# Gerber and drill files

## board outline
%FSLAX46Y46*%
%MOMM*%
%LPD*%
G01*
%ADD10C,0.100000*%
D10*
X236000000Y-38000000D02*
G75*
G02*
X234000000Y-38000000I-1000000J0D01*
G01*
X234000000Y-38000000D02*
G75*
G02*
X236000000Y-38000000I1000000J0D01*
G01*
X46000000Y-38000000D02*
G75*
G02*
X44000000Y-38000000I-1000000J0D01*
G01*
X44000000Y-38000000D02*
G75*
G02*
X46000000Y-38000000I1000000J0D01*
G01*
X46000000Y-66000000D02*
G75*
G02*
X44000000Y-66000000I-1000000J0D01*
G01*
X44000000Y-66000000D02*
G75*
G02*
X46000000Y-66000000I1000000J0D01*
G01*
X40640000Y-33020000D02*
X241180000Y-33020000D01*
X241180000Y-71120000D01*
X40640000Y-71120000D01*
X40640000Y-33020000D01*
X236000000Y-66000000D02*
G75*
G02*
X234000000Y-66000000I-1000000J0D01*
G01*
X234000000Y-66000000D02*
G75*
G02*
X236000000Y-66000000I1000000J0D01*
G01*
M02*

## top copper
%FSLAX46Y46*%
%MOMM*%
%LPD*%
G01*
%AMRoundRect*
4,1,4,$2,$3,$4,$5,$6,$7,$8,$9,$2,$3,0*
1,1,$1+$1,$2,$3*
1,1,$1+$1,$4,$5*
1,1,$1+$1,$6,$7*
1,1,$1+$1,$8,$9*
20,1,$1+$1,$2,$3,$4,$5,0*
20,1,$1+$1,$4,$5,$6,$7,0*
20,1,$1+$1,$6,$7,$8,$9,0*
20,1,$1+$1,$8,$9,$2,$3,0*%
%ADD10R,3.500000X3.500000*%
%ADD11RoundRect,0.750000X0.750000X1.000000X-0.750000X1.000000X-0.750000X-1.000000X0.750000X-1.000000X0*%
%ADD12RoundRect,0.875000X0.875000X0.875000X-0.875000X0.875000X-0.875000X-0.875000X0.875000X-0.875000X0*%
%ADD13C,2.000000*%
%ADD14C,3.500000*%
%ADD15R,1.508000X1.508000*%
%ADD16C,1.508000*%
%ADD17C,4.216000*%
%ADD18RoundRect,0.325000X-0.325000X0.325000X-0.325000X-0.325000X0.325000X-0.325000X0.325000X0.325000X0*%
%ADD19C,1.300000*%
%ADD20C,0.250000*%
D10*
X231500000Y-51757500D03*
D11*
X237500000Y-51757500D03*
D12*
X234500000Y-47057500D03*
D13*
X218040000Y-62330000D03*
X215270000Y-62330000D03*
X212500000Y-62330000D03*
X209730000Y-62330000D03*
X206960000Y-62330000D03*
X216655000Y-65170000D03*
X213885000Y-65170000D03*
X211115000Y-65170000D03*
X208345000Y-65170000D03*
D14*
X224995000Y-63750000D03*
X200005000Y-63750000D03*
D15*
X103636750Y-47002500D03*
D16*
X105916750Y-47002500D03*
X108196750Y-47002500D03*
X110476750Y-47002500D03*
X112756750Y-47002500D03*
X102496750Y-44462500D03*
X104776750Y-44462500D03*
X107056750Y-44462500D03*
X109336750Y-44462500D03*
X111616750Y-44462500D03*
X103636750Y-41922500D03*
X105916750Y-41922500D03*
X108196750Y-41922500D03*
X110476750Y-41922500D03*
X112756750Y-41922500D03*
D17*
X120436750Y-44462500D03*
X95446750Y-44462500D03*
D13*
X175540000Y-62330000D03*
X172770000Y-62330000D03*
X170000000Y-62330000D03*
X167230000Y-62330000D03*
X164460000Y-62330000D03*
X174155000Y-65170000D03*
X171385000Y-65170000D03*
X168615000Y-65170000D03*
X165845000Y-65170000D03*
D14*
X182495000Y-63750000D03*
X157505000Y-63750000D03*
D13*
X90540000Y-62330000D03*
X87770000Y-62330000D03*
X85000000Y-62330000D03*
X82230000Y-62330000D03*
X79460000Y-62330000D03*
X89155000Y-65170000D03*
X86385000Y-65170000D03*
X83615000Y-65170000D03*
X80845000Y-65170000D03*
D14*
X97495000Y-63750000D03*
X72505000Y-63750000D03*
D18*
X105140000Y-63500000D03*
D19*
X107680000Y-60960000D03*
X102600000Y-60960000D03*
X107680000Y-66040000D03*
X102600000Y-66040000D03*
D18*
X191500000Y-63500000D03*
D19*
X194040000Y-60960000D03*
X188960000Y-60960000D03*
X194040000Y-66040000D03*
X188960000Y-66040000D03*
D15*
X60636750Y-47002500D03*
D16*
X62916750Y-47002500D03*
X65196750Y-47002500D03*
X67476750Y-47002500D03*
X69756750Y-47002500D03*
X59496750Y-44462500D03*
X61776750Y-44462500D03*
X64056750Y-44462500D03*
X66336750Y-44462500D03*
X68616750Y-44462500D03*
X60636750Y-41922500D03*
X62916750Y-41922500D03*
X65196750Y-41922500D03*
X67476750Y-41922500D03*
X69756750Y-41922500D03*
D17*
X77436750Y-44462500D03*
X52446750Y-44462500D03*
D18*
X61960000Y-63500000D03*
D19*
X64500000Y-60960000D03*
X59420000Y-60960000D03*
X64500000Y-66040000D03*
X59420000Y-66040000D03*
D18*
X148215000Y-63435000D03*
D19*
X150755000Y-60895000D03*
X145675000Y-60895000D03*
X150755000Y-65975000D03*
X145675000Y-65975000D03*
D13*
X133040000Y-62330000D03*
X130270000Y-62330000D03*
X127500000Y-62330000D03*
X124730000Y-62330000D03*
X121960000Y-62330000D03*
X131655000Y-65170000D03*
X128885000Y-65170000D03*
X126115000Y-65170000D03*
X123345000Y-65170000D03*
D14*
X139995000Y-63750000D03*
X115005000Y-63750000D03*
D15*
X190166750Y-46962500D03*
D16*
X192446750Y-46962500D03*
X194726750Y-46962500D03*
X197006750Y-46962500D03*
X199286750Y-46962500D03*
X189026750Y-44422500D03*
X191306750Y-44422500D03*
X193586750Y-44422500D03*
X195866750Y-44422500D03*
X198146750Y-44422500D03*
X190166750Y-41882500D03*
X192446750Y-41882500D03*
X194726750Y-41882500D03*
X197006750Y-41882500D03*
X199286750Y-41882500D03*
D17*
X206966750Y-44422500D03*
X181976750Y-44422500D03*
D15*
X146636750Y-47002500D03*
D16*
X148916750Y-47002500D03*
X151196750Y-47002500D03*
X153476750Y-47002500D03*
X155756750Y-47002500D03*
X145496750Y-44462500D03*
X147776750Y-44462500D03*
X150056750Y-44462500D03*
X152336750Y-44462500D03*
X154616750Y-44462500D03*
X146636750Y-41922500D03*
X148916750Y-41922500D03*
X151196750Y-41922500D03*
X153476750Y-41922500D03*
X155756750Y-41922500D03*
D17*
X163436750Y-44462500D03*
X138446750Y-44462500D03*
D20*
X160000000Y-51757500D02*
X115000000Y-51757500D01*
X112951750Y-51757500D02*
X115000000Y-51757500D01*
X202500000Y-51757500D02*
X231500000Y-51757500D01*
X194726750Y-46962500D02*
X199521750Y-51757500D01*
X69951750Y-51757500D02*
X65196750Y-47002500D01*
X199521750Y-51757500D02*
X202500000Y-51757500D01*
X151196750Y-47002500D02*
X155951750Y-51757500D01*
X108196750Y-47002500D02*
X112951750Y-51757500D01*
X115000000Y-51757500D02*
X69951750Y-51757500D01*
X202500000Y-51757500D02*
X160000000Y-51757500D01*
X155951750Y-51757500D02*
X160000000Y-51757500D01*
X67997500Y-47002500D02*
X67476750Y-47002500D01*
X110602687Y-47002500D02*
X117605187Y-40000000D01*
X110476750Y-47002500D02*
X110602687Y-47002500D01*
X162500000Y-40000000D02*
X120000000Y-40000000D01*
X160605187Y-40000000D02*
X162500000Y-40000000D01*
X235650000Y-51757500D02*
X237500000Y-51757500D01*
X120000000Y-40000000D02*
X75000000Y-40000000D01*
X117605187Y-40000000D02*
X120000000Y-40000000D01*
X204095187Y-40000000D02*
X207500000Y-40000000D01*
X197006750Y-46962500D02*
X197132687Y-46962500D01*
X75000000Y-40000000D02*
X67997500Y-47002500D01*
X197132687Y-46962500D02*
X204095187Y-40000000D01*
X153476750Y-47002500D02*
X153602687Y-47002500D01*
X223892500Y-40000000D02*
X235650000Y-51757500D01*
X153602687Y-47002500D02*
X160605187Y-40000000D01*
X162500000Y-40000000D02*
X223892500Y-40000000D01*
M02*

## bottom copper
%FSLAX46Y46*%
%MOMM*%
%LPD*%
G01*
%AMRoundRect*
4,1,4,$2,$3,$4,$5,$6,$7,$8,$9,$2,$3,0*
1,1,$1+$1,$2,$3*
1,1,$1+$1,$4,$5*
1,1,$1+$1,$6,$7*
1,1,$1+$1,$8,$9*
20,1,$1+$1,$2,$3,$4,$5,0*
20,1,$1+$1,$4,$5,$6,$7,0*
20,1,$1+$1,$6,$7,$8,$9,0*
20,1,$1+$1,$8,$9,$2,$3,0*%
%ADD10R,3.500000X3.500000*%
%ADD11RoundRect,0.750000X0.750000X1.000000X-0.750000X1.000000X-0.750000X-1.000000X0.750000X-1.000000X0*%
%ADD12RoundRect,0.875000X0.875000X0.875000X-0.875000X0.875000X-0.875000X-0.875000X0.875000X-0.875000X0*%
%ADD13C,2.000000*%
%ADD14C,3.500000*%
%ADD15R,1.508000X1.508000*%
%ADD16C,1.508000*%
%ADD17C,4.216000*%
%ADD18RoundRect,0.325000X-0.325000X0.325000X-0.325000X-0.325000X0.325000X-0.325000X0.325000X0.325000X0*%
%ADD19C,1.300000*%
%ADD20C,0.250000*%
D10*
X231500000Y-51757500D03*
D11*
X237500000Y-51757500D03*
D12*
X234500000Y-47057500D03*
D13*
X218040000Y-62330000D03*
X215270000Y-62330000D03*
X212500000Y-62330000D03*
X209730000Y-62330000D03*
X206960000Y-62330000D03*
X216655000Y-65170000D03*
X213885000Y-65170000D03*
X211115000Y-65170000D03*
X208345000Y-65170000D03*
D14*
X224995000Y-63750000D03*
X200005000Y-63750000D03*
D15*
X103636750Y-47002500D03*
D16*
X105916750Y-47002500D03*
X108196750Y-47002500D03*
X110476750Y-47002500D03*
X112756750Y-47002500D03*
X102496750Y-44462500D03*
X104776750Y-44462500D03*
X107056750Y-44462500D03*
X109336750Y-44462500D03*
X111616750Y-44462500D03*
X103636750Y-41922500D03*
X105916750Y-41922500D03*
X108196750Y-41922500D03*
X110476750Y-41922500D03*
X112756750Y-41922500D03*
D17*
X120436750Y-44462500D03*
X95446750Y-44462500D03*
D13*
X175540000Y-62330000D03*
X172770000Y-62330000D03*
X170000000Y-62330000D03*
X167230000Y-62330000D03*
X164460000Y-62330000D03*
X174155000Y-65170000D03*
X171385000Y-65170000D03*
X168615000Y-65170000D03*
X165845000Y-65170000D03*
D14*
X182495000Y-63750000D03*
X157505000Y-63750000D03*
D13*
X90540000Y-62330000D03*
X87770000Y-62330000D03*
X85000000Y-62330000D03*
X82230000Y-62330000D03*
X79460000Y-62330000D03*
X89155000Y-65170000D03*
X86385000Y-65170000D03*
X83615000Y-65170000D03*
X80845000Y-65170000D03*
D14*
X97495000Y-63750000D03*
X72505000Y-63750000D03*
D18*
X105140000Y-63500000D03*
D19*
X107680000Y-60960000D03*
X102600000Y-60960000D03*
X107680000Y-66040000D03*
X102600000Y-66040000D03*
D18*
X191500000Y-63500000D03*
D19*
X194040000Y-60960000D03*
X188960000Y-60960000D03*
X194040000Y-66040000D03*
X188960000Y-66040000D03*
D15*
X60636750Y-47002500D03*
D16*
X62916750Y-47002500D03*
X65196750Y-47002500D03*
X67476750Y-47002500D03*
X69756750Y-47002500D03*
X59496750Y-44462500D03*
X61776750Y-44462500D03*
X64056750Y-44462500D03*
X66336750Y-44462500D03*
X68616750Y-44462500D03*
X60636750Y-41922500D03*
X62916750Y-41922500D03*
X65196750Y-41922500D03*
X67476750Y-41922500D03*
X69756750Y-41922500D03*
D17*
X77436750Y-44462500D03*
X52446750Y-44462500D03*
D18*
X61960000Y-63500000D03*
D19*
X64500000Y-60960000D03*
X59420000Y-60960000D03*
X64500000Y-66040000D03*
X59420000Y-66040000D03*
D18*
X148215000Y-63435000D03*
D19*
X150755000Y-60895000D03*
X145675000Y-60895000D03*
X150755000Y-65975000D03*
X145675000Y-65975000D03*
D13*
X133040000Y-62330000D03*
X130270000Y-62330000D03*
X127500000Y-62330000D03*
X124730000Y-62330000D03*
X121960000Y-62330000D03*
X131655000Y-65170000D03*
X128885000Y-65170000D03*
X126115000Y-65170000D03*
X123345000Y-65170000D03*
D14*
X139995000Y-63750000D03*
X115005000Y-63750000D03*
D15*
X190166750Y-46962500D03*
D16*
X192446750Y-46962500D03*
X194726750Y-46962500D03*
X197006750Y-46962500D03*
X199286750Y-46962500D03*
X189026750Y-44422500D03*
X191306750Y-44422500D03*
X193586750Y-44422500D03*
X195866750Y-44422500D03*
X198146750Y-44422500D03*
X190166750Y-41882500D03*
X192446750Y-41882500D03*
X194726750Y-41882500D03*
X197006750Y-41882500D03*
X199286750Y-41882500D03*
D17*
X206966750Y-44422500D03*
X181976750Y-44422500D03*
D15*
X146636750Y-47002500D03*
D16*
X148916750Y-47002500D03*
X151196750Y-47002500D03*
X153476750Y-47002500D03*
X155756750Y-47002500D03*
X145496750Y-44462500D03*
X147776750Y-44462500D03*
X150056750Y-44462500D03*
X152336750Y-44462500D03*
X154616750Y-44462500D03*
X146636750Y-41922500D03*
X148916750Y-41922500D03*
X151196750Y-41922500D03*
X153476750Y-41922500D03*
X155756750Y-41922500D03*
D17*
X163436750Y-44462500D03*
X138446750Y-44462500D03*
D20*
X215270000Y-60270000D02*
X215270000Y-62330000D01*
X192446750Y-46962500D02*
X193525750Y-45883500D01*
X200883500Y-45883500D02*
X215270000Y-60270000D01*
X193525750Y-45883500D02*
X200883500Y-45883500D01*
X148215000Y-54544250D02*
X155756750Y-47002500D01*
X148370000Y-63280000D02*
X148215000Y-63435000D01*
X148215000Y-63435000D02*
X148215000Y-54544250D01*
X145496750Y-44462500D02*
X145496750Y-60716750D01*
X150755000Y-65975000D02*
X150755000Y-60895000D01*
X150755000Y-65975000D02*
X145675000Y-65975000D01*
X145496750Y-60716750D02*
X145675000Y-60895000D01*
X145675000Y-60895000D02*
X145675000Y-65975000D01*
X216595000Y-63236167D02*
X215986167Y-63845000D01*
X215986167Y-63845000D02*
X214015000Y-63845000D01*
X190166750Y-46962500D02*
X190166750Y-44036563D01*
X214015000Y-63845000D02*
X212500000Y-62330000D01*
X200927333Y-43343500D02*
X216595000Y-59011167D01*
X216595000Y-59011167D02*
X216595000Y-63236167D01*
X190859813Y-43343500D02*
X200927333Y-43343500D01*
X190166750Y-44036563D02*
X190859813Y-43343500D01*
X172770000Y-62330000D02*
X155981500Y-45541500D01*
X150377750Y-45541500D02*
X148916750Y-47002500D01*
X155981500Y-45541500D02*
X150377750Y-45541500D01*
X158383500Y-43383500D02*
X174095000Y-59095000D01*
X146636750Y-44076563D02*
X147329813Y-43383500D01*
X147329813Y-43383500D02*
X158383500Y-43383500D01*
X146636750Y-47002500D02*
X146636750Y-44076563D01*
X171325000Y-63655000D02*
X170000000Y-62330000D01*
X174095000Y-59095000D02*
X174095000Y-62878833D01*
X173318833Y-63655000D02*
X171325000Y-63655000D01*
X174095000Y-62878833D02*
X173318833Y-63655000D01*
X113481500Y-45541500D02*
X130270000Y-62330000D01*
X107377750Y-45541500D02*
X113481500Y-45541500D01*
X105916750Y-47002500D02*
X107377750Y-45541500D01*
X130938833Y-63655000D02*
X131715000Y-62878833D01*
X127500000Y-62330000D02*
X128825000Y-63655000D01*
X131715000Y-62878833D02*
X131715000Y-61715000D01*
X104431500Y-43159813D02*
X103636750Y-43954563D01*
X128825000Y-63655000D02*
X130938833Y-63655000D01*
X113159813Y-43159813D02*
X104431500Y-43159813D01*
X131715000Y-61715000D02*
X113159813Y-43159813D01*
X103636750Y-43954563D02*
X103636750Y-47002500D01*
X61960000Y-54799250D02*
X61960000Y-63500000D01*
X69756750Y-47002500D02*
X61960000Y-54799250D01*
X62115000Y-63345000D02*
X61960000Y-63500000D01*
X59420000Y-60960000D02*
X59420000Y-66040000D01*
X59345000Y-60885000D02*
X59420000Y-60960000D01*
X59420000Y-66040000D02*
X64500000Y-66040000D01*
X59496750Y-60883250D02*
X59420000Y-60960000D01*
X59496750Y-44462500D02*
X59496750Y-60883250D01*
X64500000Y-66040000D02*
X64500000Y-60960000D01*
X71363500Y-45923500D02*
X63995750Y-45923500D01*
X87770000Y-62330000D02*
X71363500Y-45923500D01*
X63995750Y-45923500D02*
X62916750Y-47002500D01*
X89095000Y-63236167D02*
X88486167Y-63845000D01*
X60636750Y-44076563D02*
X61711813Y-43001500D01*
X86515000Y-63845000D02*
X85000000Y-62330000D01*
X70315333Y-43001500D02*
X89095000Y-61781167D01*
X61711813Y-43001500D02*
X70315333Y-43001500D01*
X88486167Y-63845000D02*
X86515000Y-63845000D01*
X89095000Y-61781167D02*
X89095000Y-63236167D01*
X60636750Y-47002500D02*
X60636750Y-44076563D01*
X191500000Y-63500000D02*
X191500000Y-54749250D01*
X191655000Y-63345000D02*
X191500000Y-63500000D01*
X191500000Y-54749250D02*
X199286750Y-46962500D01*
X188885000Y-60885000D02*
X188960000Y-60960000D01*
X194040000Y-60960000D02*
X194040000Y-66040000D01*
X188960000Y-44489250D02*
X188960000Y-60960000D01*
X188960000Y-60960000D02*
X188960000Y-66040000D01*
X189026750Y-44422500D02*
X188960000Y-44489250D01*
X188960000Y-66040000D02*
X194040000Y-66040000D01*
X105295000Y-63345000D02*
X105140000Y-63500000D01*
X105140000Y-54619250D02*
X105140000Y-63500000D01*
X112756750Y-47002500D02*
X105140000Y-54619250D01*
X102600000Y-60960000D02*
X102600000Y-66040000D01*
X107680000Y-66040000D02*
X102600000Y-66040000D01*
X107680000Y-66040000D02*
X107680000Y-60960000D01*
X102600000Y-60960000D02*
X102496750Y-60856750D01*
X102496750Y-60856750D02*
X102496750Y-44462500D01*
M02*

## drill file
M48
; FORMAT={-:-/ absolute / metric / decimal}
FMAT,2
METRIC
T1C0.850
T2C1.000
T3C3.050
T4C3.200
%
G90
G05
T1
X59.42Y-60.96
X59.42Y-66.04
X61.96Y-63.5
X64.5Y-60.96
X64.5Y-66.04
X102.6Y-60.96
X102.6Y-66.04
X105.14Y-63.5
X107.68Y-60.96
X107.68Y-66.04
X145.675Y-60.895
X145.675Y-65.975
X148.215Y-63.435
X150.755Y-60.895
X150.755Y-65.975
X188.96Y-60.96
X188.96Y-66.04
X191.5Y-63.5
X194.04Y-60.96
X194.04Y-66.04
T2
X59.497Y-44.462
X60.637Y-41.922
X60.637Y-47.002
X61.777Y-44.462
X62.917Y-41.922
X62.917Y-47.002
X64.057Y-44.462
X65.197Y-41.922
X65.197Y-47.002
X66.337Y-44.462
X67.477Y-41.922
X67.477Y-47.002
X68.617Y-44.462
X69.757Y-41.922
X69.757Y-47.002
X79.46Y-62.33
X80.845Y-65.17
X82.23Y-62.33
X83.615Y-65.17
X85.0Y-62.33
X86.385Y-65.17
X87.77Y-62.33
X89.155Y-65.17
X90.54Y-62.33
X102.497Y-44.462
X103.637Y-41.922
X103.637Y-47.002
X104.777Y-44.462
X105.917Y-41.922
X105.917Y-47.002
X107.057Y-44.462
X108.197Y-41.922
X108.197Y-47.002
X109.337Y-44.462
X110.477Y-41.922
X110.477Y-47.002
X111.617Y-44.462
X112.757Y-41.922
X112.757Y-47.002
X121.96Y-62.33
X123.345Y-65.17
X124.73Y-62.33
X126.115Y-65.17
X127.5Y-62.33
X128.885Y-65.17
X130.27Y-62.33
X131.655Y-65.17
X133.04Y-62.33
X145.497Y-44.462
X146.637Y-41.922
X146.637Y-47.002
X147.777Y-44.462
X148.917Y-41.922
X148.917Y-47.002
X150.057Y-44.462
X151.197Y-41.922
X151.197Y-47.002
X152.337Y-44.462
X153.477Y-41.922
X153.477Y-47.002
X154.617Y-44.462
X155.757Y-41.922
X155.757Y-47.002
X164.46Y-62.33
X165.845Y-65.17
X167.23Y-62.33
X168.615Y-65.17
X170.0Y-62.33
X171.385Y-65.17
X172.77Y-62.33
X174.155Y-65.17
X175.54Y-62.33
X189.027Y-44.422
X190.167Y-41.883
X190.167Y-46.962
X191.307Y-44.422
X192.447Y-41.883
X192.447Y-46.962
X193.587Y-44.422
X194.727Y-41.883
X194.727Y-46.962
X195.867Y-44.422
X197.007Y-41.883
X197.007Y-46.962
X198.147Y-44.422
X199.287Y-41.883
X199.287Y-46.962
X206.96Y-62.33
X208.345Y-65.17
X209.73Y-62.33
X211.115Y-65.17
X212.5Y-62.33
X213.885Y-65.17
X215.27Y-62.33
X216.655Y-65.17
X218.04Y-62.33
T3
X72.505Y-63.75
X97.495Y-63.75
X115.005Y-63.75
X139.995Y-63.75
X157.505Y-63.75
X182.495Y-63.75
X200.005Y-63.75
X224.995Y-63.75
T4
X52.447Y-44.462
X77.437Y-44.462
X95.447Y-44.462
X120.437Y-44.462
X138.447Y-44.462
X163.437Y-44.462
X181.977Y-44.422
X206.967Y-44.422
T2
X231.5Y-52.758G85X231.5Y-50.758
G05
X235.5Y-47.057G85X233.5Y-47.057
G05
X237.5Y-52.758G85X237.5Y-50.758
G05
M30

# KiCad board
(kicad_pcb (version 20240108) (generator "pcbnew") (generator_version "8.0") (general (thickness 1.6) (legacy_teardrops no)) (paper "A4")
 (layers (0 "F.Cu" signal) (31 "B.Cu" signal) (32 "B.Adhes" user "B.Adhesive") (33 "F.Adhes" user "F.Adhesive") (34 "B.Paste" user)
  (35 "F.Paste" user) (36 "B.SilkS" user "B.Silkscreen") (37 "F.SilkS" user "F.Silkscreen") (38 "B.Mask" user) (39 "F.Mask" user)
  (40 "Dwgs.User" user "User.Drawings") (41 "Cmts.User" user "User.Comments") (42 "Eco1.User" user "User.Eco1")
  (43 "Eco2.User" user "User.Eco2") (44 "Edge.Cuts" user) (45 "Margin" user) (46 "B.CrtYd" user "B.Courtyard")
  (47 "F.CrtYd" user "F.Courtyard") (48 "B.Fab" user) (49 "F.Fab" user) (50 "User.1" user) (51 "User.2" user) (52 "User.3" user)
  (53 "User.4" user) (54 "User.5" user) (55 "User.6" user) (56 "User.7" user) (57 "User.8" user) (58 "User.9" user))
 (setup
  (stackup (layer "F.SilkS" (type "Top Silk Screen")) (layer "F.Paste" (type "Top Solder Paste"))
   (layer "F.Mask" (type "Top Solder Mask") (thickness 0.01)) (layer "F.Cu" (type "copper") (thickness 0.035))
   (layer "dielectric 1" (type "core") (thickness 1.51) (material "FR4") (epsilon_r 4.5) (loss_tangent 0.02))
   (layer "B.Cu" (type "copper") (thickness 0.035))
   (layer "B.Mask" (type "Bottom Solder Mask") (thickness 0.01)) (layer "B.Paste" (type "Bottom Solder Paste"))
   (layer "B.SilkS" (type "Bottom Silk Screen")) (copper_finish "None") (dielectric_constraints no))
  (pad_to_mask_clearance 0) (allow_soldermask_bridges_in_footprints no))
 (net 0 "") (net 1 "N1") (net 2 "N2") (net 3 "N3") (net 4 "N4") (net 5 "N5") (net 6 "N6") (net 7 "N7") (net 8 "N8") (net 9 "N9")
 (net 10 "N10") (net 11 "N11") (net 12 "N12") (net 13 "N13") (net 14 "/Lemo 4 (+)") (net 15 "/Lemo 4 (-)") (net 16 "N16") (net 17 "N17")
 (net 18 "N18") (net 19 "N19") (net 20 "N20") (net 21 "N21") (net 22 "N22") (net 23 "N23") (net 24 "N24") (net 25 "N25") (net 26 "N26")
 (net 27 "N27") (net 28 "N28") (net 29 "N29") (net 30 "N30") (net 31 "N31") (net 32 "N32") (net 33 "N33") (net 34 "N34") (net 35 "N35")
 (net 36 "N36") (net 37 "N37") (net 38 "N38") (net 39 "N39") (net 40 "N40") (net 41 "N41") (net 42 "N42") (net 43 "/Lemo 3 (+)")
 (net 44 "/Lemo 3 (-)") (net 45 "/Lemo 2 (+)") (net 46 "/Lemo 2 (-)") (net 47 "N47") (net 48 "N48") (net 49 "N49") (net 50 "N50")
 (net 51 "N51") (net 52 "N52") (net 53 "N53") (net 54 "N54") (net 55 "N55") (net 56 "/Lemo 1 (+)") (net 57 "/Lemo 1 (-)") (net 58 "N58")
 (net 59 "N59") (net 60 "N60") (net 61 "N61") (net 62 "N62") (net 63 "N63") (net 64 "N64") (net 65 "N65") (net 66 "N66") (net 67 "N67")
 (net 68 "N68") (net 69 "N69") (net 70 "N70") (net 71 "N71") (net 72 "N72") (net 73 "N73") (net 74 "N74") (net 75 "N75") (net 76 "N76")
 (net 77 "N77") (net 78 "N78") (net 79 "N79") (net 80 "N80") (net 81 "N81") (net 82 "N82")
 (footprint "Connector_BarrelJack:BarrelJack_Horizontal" (layer "F.Cu") (at 231.5 51.7575 180)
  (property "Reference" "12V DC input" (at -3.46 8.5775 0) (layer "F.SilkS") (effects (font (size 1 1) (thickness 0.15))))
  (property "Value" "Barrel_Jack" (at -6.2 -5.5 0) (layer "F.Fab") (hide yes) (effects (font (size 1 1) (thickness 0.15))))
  (pad "1" thru_hole rect (at 0 0 180) (size 3.5 3.5) (drill oval 1 3) (layers "*.Cu" "*.Mask") (remove_unused_layers no) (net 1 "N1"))
  (pad "2" thru_hole roundrect (at -6 0 180) (size 3 3.5) (drill oval 1 3) (layers "*.Cu" "*.Mask") (remove_unused_layers no)
   (roundrect_rratio 0.25) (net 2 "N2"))
  (pad "3" thru_hole roundrect (at -3 4.7 180) (size 3.5 3.5) (drill oval 3 1) (layers "*.Cu" "*.Mask") (remove_unused_layers no)
   (roundrect_rratio 0.25)))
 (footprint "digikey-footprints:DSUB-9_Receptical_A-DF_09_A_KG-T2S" (layer "F.Cu") (at 212.5 63.75 180)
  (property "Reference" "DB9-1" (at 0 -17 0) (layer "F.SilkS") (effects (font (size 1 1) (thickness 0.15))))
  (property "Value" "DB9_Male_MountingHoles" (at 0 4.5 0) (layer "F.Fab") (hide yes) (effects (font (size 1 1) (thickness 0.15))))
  (pad "1" thru_hole circle (at -5.54 1.42 180) (size 2 2) (drill 1) (layers "*.Cu" "*.Mask") (remove_unused_layers no) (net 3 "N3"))
  (pad "2" thru_hole circle (at -2.77 1.42 180) (size 2 2) (drill 1) (layers "*.Cu" "*.Mask") (remove_unused_layers no) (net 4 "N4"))
  (pad "3" thru_hole circle (at 0 1.42 180) (size 2 2) (drill 1) (layers "*.Cu" "*.Mask") (remove_unused_layers no) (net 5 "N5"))
  (pad "4" thru_hole circle (at 2.77 1.42 180) (size 2 2) (drill 1) (layers "*.Cu" "*.Mask") (remove_unused_layers no) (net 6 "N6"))
  (pad "5" thru_hole circle (at 5.54 1.42 180) (size 2 2) (drill 1) (layers "*.Cu" "*.Mask") (remove_unused_layers no) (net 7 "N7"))
  (pad "6" thru_hole circle (at -4.155 -1.42 180) (size 2 2) (drill 1) (layers "*.Cu" "*.Mask") (remove_unused_layers no) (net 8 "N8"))
  (pad "7" thru_hole circle (at -1.385 -1.42 180) (size 2 2) (drill 1) (layers "*.Cu" "*.Mask") (remove_unused_layers no) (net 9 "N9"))
  (pad "8" thru_hole circle (at 1.385 -1.42 180) (size 2 2) (drill 1) (layers "*.Cu" "*.Mask") (remove_unused_layers no) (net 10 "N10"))
  (pad "9" thru_hole circle (at 4.155 -1.42 180) (size 2 2) (drill 1) (layers "*.Cu" "*.Mask") (remove_unused_layers no) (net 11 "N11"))
  (pad "10" thru_hole circle (at -12.495 0 180) (size 3.5 3.5) (drill 3.05) (layers "*.Cu" "*.Mask") (remove_unused_layers no))
  (pad "10" thru_hole circle (at 12.495 0 180) (size 3.5 3.5) (drill 3.05) (layers "*.Cu" "*.Mask") (remove_unused_layers no)))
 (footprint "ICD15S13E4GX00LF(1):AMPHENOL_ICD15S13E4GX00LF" (layer "F.Cu") (at 107.94175 44.4625 180)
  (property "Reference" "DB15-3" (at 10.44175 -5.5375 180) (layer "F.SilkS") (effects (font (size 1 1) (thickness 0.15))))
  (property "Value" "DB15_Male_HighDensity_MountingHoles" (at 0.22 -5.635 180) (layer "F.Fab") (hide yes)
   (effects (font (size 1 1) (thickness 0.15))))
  (pad "1" thru_hole rect (at 4.305 -2.54 180) (size 1.508 1.508) (drill 1) (layers "*.Cu" "*.Mask") (remove_unused_layers no)
   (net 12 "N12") (solder_mask_margin 0.102))
  (pad "2" thru_hole circle (at 2.025 -2.54 180) (size 1.508 1.508) (drill 1) (layers "*.Cu" "*.Mask") (remove_unused_layers no)
   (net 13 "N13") (solder_mask_margin 0.102))
  (pad "3" thru_hole circle (at -0.255 -2.54 180) (size 1.508 1.508) (drill 1) (layers "*.Cu" "*.Mask") (remove_unused_layers no)
   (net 1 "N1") (solder_mask_margin 0.102))
  (pad "4" thru_hole circle (at -2.535 -2.54 180) (size 1.508 1.508) (drill 1) (layers "*.Cu" "*.Mask") (remove_unused_layers no)
   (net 2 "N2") (solder_mask_margin 0.102))
  (pad "5" thru_hole circle (at -4.815 -2.54 180) (size 1.508 1.508) (drill 1) (layers "*.Cu" "*.Mask") (remove_unused_layers no)
   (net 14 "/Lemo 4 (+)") (solder_mask_margin 0.102))
  (pad "6" thru_hole circle (at 5.445 0 180) (size 1.508 1.508) (drill 1) (layers "*.Cu" "*.Mask") (remove_unused_layers no)
   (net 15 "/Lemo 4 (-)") (solder_mask_margin 0.102))
  (pad "7" thru_hole circle (at 3.165 0 180) (size 1.508 1.508) (drill 1) (layers "*.Cu" "*.Mask") (remove_unused_layers no) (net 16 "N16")
   (solder_mask_margin 0.102))
  (pad "8" thru_hole circle (at 0.885 0 180) (size 1.508 1.508) (drill 1) (layers "*.Cu" "*.Mask") (remove_unused_layers no) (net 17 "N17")
   (solder_mask_margin 0.102))
  (pad "9" thru_hole circle (at -1.395 0 180) (size 1.508 1.508) (drill 1) (layers "*.Cu" "*.Mask") (remove_unused_layers no) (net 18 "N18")
   (solder_mask_margin 0.102))
  (pad "10" thru_hole circle (at -3.675 0 180) (size 1.508 1.508) (drill 1) (layers "*.Cu" "*.Mask") (remove_unused_layers no)
   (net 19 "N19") (solder_mask_margin 0.102))
  (pad "11" thru_hole circle (at 4.305 2.54 180) (size 1.508 1.508) (drill 1) (layers "*.Cu" "*.Mask") (remove_unused_layers no)
   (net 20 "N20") (solder_mask_margin 0.102))
  (pad "12" thru_hole circle (at 2.025 2.54 180) (size 1.508 1.508) (drill 1) (layers "*.Cu" "*.Mask") (remove_unused_layers no)
   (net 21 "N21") (solder_mask_margin 0.102))
  (pad "13" thru_hole circle (at -0.255 2.54 180) (size 1.508 1.508) (drill 1) (layers "*.Cu" "*.Mask") (remove_unused_layers no)
   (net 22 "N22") (solder_mask_margin 0.102))
  (pad "14" thru_hole circle (at -2.535 2.54 180) (size 1.508 1.508) (drill 1) (layers "*.Cu" "*.Mask") (remove_unused_layers no)
   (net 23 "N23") (solder_mask_margin 0.102))
  (pad "15" thru_hole circle (at -4.815 2.54 180) (size 1.508 1.508) (drill 1) (layers "*.Cu" "*.Mask") (remove_unused_layers no)
   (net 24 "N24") (solder_mask_margin 0.102))
  (pad "S1" thru_hole circle (at -12.495 0 180) (size 4.216 4.216) (drill 3.2) (layers "*.Cu" "*.Mask") (remove_unused_layers no)
   (solder_mask_margin 0.102))
  (pad "S2" thru_hole circle (at 12.495 0 180) (size 4.216 4.216) (drill 3.2) (layers "*.Cu" "*.Mask") (remove_unused_layers no)
   (solder_mask_margin 0.102)))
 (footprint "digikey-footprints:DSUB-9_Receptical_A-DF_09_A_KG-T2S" (layer "F.Cu") (at 170 63.75 180)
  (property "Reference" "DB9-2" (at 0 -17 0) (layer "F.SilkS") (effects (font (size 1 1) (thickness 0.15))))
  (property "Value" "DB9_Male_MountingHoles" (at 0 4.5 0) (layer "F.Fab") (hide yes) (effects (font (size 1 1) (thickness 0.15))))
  (pad "1" thru_hole circle (at -5.54 1.42 180) (size 2 2) (drill 1) (layers "*.Cu" "*.Mask") (remove_unused_layers no) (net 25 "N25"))
  (pad "2" thru_hole circle (at -2.77 1.42 180) (size 2 2) (drill 1) (layers "*.Cu" "*.Mask") (remove_unused_layers no) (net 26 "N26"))
  (pad "3" thru_hole circle (at 0 1.42 180) (size 2 2) (drill 1) (layers "*.Cu" "*.Mask") (remove_unused_layers no) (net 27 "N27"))
  (pad "4" thru_hole circle (at 2.77 1.42 180) (size 2 2) (drill 1) (layers "*.Cu" "*.Mask") (remove_unused_layers no) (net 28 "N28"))
  (pad "5" thru_hole circle (at 5.54 1.42 180) (size 2 2) (drill 1) (layers "*.Cu" "*.Mask") (remove_unused_layers no) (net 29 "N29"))
  (pad "6" thru_hole circle (at -4.155 -1.42 180) (size 2 2) (drill 1) (layers "*.Cu" "*.Mask") (remove_unused_layers no) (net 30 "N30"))
  (pad "7" thru_hole circle (at -1.385 -1.42 180) (size 2 2) (drill 1) (layers "*.Cu" "*.Mask") (remove_unused_layers no) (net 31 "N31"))
  (pad "8" thru_hole circle (at 1.385 -1.42 180) (size 2 2) (drill 1) (layers "*.Cu" "*.Mask") (remove_unused_layers no) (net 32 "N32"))
  (pad "9" thru_hole circle (at 4.155 -1.42 180) (size 2 2) (drill 1) (layers "*.Cu" "*.Mask") (remove_unused_layers no) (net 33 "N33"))
  (pad "10" thru_hole circle (at -12.495 0 180) (size 3.5 3.5) (drill 3.05) (layers "*.Cu" "*.Mask") (remove_unused_layers no))
  (pad "10" thru_hole circle (at 12.495 0 180) (size 3.5 3.5) (drill 3.05) (layers "*.Cu" "*.Mask") (remove_unused_layers no)))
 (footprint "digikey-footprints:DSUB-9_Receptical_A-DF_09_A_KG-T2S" (layer "F.Cu") (at 85 63.75 180)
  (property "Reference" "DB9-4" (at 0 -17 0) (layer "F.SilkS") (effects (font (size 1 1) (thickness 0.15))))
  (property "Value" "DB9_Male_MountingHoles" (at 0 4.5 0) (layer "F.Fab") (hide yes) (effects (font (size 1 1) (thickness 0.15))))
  (pad "1" thru_hole circle (at -5.54 1.42 180) (size 2 2) (drill 1) (layers "*.Cu" "*.Mask") (remove_unused_layers no) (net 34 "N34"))
  (pad "2" thru_hole circle (at -2.77 1.42 180) (size 2 2) (drill 1) (layers "*.Cu" "*.Mask") (remove_unused_layers no) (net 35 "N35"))
  (pad "3" thru_hole circle (at 0 1.42 180) (size 2 2) (drill 1) (layers "*.Cu" "*.Mask") (remove_unused_layers no) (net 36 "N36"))
  (pad "4" thru_hole circle (at 2.77 1.42 180) (size 2 2) (drill 1) (layers "*.Cu" "*.Mask") (remove_unused_layers no) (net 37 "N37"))
  (pad "5" thru_hole circle (at 5.54 1.42 180) (size 2 2) (drill 1) (layers "*.Cu" "*.Mask") (remove_unused_layers no) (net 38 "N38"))
  (pad "6" thru_hole circle (at -4.155 -1.42 180) (size 2 2) (drill 1) (layers "*.Cu" "*.Mask") (remove_unused_layers no) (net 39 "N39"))
  (pad "7" thru_hole circle (at -1.385 -1.42 180) (size 2 2) (drill 1) (layers "*.Cu" "*.Mask") (remove_unused_layers no) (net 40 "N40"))
  (pad "8" thru_hole circle (at 1.385 -1.42 180) (size 2 2) (drill 1) (layers "*.Cu" "*.Mask") (remove_unused_layers no) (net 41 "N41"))
  (pad "9" thru_hole circle (at 4.155 -1.42 180) (size 2 2) (drill 1) (layers "*.Cu" "*.Mask") (remove_unused_layers no) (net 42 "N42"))
  (pad "10" thru_hole circle (at -12.495 0 180) (size 3.5 3.5) (drill 3.05) (layers "*.Cu" "*.Mask") (remove_unused_layers no))
  (pad "10" thru_hole circle (at 12.495 0 180) (size 3.5 3.5) (drill 3.05) (layers "*.Cu" "*.Mask") (remove_unused_layers no)))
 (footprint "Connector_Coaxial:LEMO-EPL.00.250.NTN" (layer "F.Cu") (at 105.14 63.5 -90)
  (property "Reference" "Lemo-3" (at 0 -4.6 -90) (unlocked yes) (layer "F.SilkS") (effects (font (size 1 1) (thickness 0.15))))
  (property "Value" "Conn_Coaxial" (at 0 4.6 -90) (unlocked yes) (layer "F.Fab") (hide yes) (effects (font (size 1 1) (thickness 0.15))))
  (pad "1" thru_hole roundrect (at 0 0 270) (size 1.3 1.3) (drill 0.85) (layers "*.Cu" "*.Mask") (remove_unused_layers no)
   (roundrect_rratio 0.25) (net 14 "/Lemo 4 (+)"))
  (pad "2" thru_hole circle (at -2.54 -2.54 270) (size 1.3 1.3) (drill 0.85) (layers "*.Cu" "*.Mask") (remove_unused_layers no)
   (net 15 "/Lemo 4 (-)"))
  (pad "2" thru_hole circle (at -2.54 2.54 270) (size 1.3 1.3) (drill 0.85) (layers "*.Cu" "*.Mask") (remove_unused_layers no)
   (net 15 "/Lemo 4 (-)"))
  (pad "2" thru_hole circle (at 2.54 -2.54 270) (size 1.3 1.3) (drill 0.85) (layers "*.Cu" "*.Mask") (remove_unused_layers no)
   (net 15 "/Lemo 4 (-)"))
  (pad "2" thru_hole circle (at 2.54 2.54 270) (size 1.3 1.3) (drill 0.85) (layers "*.Cu" "*.Mask") (remove_unused_layers no)
   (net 15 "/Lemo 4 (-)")))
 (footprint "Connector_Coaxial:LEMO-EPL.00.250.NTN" (layer "F.Cu") (at 191.5 63.5 -90)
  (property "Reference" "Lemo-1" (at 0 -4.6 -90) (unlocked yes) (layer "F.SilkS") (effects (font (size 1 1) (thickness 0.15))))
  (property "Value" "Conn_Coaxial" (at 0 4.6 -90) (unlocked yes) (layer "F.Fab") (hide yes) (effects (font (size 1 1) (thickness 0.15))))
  (pad "1" thru_hole roundrect (at 0 0 270) (size 1.3 1.3) (drill 0.85) (layers "*.Cu" "*.Mask") (remove_unused_layers no)
   (roundrect_rratio 0.25) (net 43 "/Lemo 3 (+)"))
  (pad "2" thru_hole circle (at -2.54 -2.54 270) (size 1.3 1.3) (drill 0.85) (layers "*.Cu" "*.Mask") (remove_unused_layers no)
   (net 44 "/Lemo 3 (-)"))
  (pad "2" thru_hole circle (at -2.54 2.54 270) (size 1.3 1.3) (drill 0.85) (layers "*.Cu" "*.Mask") (remove_unused_layers no)
   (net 44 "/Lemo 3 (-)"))
  (pad "2" thru_hole circle (at 2.54 -2.54 270) (size 1.3 1.3) (drill 0.85) (layers "*.Cu" "*.Mask") (remove_unused_layers no)
   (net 44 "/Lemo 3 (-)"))
  (pad "2" thru_hole circle (at 2.54 2.54 270) (size 1.3 1.3) (drill 0.85) (layers "*.Cu" "*.Mask") (remove_unused_layers no)
   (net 44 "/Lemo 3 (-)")))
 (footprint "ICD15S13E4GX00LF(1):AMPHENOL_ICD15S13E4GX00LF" (layer "F.Cu") (at 64.94175 44.4625 180)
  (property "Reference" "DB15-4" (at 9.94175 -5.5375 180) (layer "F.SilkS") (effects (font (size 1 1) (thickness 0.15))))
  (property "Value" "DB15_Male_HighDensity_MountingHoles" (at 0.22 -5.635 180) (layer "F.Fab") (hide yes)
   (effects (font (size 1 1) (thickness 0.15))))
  (pad "1" thru_hole rect (at 4.305 -2.54 180) (size 1.508 1.508) (drill 1) (layers "*.Cu" "*.Mask") (remove_unused_layers no)
   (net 36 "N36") (solder_mask_margin 0.102))
  (pad "2" thru_hole circle (at 2.025 -2.54 180) (size 1.508 1.508) (drill 1) (layers "*.Cu" "*.Mask") (remove_unused_layers no)
   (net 35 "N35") (solder_mask_margin 0.102))
  (pad "3" thru_hole circle (at -0.255 -2.54 180) (size 1.508 1.508) (drill 1) (layers "*.Cu" "*.Mask") (remove_unused_layers no)
   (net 1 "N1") (solder_mask_margin 0.102))
  (pad "4" thru_hole circle (at -2.535 -2.54 180) (size 1.508 1.508) (drill 1) (layers "*.Cu" "*.Mask") (remove_unused_layers no)
   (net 2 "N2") (solder_mask_margin 0.102))
  (pad "5" thru_hole circle (at -4.815 -2.54 180) (size 1.508 1.508) (drill 1) (layers "*.Cu" "*.Mask") (remove_unused_layers no)
   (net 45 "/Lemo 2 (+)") (solder_mask_margin 0.102))
  (pad "6" thru_hole circle (at 5.445 0 180) (size 1.508 1.508) (drill 1) (layers "*.Cu" "*.Mask") (remove_unused_layers no)
   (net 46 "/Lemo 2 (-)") (solder_mask_margin 0.102))
  (pad "7" thru_hole circle (at 3.165 0 180) (size 1.508 1.508) (drill 1) (layers "*.Cu" "*.Mask") (remove_unused_layers no) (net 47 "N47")
   (solder_mask_margin 0.102))
  (pad "8" thru_hole circle (at 0.885 0 180) (size 1.508 1.508) (drill 1) (layers "*.Cu" "*.Mask") (remove_unused_layers no) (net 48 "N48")
   (solder_mask_margin 0.102))
  (pad "9" thru_hole circle (at -1.395 0 180) (size 1.508 1.508) (drill 1) (layers "*.Cu" "*.Mask") (remove_unused_layers no) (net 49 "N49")
   (solder_mask_margin 0.102))
  (pad "10" thru_hole circle (at -3.675 0 180) (size 1.508 1.508) (drill 1) (layers "*.Cu" "*.Mask") (remove_unused_layers no)
   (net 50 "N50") (solder_mask_margin 0.102))
  (pad "11" thru_hole circle (at 4.305 2.54 180) (size 1.508 1.508) (drill 1) (layers "*.Cu" "*.Mask") (remove_unused_layers no)
   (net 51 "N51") (solder_mask_margin 0.102))
  (pad "12" thru_hole circle (at 2.025 2.54 180) (size 1.508 1.508) (drill 1) (layers "*.Cu" "*.Mask") (remove_unused_layers no)
   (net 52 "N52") (solder_mask_margin 0.102))
  (pad "13" thru_hole circle (at -0.255 2.54 180) (size 1.508 1.508) (drill 1) (layers "*.Cu" "*.Mask") (remove_unused_layers no)
   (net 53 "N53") (solder_mask_margin 0.102))
  (pad "14" thru_hole circle (at -2.535 2.54 180) (size 1.508 1.508) (drill 1) (layers "*.Cu" "*.Mask") (remove_unused_layers no)
   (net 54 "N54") (solder_mask_margin 0.102))
  (pad "15" thru_hole circle (at -4.815 2.54 180) (size 1.508 1.508) (drill 1) (layers "*.Cu" "*.Mask") (remove_unused_layers no)
   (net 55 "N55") (solder_mask_margin 0.102))
  (pad "S1" thru_hole circle (at -12.495 0 180) (size 4.216 4.216) (drill 3.2) (layers "*.Cu" "*.Mask") (remove_unused_layers no)
   (solder_mask_margin 0.102))
  (pad "S2" thru_hole circle (at 12.495 0 180) (size 4.216 4.216) (drill 3.2) (layers "*.Cu" "*.Mask") (remove_unused_layers no)
   (solder_mask_margin 0.102)))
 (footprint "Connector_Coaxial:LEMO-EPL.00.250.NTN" (layer "F.Cu") (at 61.96 63.5 -90)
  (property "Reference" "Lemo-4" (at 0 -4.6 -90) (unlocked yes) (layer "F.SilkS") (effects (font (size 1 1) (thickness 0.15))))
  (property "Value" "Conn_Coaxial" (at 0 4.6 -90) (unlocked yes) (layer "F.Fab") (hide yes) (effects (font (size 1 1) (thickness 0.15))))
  (pad "1" thru_hole roundrect (at 0 0 270) (size 1.3 1.3) (drill 0.85) (layers "*.Cu" "*.Mask") (remove_unused_layers no)
   (roundrect_rratio 0.25) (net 45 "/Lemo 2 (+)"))
  (pad "2" thru_hole circle (at -2.54 -2.54 270) (size 1.3 1.3) (drill 0.85) (layers "*.Cu" "*.Mask") (remove_unused_layers no)
   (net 46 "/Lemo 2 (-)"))
  (pad "2" thru_hole circle (at -2.54 2.54 270) (size 1.3 1.3) (drill 0.85) (layers "*.Cu" "*.Mask") (remove_unused_layers no)
   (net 46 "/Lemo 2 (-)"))
  (pad "2" thru_hole circle (at 2.54 -2.54 270) (size 1.3 1.3) (drill 0.85) (layers "*.Cu" "*.Mask") (remove_unused_layers no)
   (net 46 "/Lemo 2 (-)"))
  (pad "2" thru_hole circle (at 2.54 2.54 270) (size 1.3 1.3) (drill 0.85) (layers "*.Cu" "*.Mask") (remove_unused_layers no)
   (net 46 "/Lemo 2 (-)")))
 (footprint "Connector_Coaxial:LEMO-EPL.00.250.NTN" (layer "F.Cu") (at 148.215 63.435 -90)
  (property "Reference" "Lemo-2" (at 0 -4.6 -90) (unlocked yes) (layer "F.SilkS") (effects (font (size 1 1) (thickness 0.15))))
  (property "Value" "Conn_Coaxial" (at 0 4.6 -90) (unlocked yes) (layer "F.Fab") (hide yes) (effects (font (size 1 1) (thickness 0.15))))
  (pad "1" thru_hole roundrect (at 0 0 270) (size 1.3 1.3) (drill 0.85) (layers "*.Cu" "*.Mask") (remove_unused_layers no)
   (roundrect_rratio 0.25) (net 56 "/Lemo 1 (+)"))
  (pad "2" thru_hole circle (at -2.54 -2.54 270) (size 1.3 1.3) (drill 0.85) (layers "*.Cu" "*.Mask") (remove_unused_layers no)
   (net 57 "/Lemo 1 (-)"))
  (pad "2" thru_hole circle (at -2.54 2.54 270) (size 1.3 1.3) (drill 0.85) (layers "*.Cu" "*.Mask") (remove_unused_layers no)
   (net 57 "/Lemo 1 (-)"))
  (pad "2" thru_hole circle (at 2.54 -2.54 270) (size 1.3 1.3) (drill 0.85) (layers "*.Cu" "*.Mask") (remove_unused_layers no)
   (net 57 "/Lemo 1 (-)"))
  (pad "2" thru_hole circle (at 2.54 2.54 270) (size 1.3 1.3) (drill 0.85) (layers "*.Cu" "*.Mask") (remove_unused_layers no)
   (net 57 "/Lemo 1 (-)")))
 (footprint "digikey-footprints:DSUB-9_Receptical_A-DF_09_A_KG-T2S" (layer "F.Cu") (at 127.5 63.75 180)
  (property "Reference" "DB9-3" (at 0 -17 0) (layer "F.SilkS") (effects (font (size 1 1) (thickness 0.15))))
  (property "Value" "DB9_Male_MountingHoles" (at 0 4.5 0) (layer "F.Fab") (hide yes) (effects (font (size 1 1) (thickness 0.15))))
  (pad "1" thru_hole circle (at -5.54 1.42 180) (size 2 2) (drill 1) (layers "*.Cu" "*.Mask") (remove_unused_layers no) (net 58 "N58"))
  (pad "2" thru_hole circle (at -2.77 1.42 180) (size 2 2) (drill 1) (layers "*.Cu" "*.Mask") (remove_unused_layers no) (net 13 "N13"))
  (pad "3" thru_hole circle (at 0 1.42 180) (size 2 2) (drill 1) (layers "*.Cu" "*.Mask") (remove_unused_layers no) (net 12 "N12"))
  (pad "4" thru_hole circle (at 2.77 1.42 180) (size 2 2) (drill 1) (layers "*.Cu" "*.Mask") (remove_unused_layers no) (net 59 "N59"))
  (pad "5" thru_hole circle (at 5.54 1.42 180) (size 2 2) (drill 1) (layers "*.Cu" "*.Mask") (remove_unused_layers no) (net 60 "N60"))
  (pad "6" thru_hole circle (at -4.155 -1.42 180) (size 2 2) (drill 1) (layers "*.Cu" "*.Mask") (remove_unused_layers no) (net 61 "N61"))
  (pad "7" thru_hole circle (at -1.385 -1.42 180) (size 2 2) (drill 1) (layers "*.Cu" "*.Mask") (remove_unused_layers no) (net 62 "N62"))
  (pad "8" thru_hole circle (at 1.385 -1.42 180) (size 2 2) (drill 1) (layers "*.Cu" "*.Mask") (remove_unused_layers no) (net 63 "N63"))
  (pad "9" thru_hole circle (at 4.155 -1.42 180) (size 2 2) (drill 1) (layers "*.Cu" "*.Mask") (remove_unused_layers no) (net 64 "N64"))
  (pad "10" thru_hole circle (at -12.495 0 180) (size 3.5 3.5) (drill 3.05) (layers "*.Cu" "*.Mask") (remove_unused_layers no))
  (pad "10" thru_hole circle (at 12.495 0 180) (size 3.5 3.5) (drill 3.05) (layers "*.Cu" "*.Mask") (remove_unused_layers no)))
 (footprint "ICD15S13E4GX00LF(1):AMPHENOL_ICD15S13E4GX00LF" (layer "F.Cu") (at 194.47175 44.4225 180)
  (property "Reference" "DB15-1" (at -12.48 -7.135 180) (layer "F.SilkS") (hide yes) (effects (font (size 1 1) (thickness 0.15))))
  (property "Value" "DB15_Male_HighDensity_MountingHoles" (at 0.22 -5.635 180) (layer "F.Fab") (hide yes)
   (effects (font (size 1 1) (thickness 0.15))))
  (pad "1" thru_hole rect (at 4.305 -2.54 180) (size 1.508 1.508) (drill 1) (layers "*.Cu" "*.Mask") (remove_unused_layers no) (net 5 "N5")
   (solder_mask_margin 0.102))
  (pad "2" thru_hole circle (at 2.025 -2.54 180) (size 1.508 1.508) (drill 1) (layers "*.Cu" "*.Mask") (remove_unused_layers no)
   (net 4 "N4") (solder_mask_margin 0.102))
  (pad "3" thru_hole circle (at -0.255 -2.54 180) (size 1.508 1.508) (drill 1) (layers "*.Cu" "*.Mask") (remove_unused_layers no)
   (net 1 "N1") (solder_mask_margin 0.102))
  (pad "4" thru_hole circle (at -2.535 -2.54 180) (size 1.508 1.508) (drill 1) (layers "*.Cu" "*.Mask") (remove_unused_layers no)
   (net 2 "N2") (solder_mask_margin 0.102))
  (pad "5" thru_hole circle (at -4.815 -2.54 180) (size 1.508 1.508) (drill 1) (layers "*.Cu" "*.Mask") (remove_unused_layers no)
   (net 43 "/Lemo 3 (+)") (solder_mask_margin 0.102))
  (pad "6" thru_hole circle (at 5.445 0 180) (size 1.508 1.508) (drill 1) (layers "*.Cu" "*.Mask") (remove_unused_layers no)
   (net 44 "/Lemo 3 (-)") (solder_mask_margin 0.102))
  (pad "7" thru_hole circle (at 3.165 0 180) (size 1.508 1.508) (drill 1) (layers "*.Cu" "*.Mask") (remove_unused_layers no) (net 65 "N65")
   (solder_mask_margin 0.102))
  (pad "8" thru_hole circle (at 0.885 0 180) (size 1.508 1.508) (drill 1) (layers "*.Cu" "*.Mask") (remove_unused_layers no) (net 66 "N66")
   (solder_mask_margin 0.102))
  (pad "9" thru_hole circle (at -1.395 0 180) (size 1.508 1.508) (drill 1) (layers "*.Cu" "*.Mask") (remove_unused_layers no) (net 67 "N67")
   (solder_mask_margin 0.102))
  (pad "10" thru_hole circle (at -3.675 0 180) (size 1.508 1.508) (drill 1) (layers "*.Cu" "*.Mask") (remove_unused_layers no)
   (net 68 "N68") (solder_mask_margin 0.102))
  (pad "11" thru_hole circle (at 4.305 2.54 180) (size 1.508 1.508) (drill 1) (layers "*.Cu" "*.Mask") (remove_unused_layers no)
   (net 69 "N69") (solder_mask_margin 0.102))
  (pad "12" thru_hole circle (at 2.025 2.54 180) (size 1.508 1.508) (drill 1) (layers "*.Cu" "*.Mask") (remove_unused_layers no)
   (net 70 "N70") (solder_mask_margin 0.102))
  (pad "13" thru_hole circle (at -0.255 2.54 180) (size 1.508 1.508) (drill 1) (layers "*.Cu" "*.Mask") (remove_unused_layers no)
   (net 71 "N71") (solder_mask_margin 0.102))
  (pad "14" thru_hole circle (at -2.535 2.54 180) (size 1.508 1.508) (drill 1) (layers "*.Cu" "*.Mask") (remove_unused_layers no)
   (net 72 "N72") (solder_mask_margin 0.102))
  (pad "15" thru_hole circle (at -4.815 2.54 180) (size 1.508 1.508) (drill 1) (layers "*.Cu" "*.Mask") (remove_unused_layers no)
   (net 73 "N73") (solder_mask_margin 0.102))
  (pad "S1" thru_hole circle (at -12.495 0 180) (size 4.216 4.216) (drill 3.2) (layers "*.Cu" "*.Mask") (remove_unused_layers no)
   (solder_mask_margin 0.102))
  (pad "S2" thru_hole circle (at 12.495 0 180) (size 4.216 4.216) (drill 3.2) (layers "*.Cu" "*.Mask") (remove_unused_layers no)
   (solder_mask_margin 0.102)))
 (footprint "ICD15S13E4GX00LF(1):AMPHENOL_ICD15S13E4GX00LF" (layer "F.Cu") (at 150.94175 44.4625 180)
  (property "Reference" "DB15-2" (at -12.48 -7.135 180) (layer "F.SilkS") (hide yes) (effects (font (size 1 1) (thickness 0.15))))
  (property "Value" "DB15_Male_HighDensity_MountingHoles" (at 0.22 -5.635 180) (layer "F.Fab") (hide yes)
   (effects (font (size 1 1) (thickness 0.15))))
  (pad "1" thru_hole rect (at 4.305 -2.54 180) (size 1.508 1.508) (drill 1) (layers "*.Cu" "*.Mask") (remove_unused_layers no)
   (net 27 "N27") (solder_mask_margin 0.102))
  (pad "2" thru_hole circle (at 2.025 -2.54 180) (size 1.508 1.508) (drill 1) (layers "*.Cu" "*.Mask") (remove_unused_layers no)
   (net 26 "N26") (solder_mask_margin 0.102))
  (pad "3" thru_hole circle (at -0.255 -2.54 180) (size 1.508 1.508) (drill 1) (layers "*.Cu" "*.Mask") (remove_unused_layers no)
   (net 1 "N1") (solder_mask_margin 0.102))
  (pad "4" thru_hole circle (at -2.535 -2.54 180) (size 1.508 1.508) (drill 1) (layers "*.Cu" "*.Mask") (remove_unused_layers no)
   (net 2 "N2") (solder_mask_margin 0.102))
  (pad "5" thru_hole circle (at -4.815 -2.54 180) (size 1.508 1.508) (drill 1) (layers "*.Cu" "*.Mask") (remove_unused_layers no)
   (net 56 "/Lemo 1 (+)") (solder_mask_margin 0.102))
  (pad "6" thru_hole circle (at 5.445 0 180) (size 1.508 1.508) (drill 1) (layers "*.Cu" "*.Mask") (remove_unused_layers no)
   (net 57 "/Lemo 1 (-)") (solder_mask_margin 0.102))
  (pad "7" thru_hole circle (at 3.165 0 180) (size 1.508 1.508) (drill 1) (layers "*.Cu" "*.Mask") (remove_unused_layers no) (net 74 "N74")
   (solder_mask_margin 0.102))
  (pad "8" thru_hole circle (at 0.885 0 180) (size 1.508 1.508) (drill 1) (layers "*.Cu" "*.Mask") (remove_unused_layers no) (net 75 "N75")
   (solder_mask_margin 0.102))
  (pad "9" thru_hole circle (at -1.395 0 180) (size 1.508 1.508) (drill 1) (layers "*.Cu" "*.Mask") (remove_unused_layers no) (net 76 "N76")
   (solder_mask_margin 0.102))
  (pad "10" thru_hole circle (at -3.675 0 180) (size 1.508 1.508) (drill 1) (layers "*.Cu" "*.Mask") (remove_unused_layers no)
   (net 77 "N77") (solder_mask_margin 0.102))
  (pad "11" thru_hole circle (at 4.305 2.54 180) (size 1.508 1.508) (drill 1) (layers "*.Cu" "*.Mask") (remove_unused_layers no)
   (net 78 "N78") (solder_mask_margin 0.102))
  (pad "12" thru_hole circle (at 2.025 2.54 180) (size 1.508 1.508) (drill 1) (layers "*.Cu" "*.Mask") (remove_unused_layers no)
   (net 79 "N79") (solder_mask_margin 0.102))
  (pad "13" thru_hole circle (at -0.255 2.54 180) (size 1.508 1.508) (drill 1) (layers "*.Cu" "*.Mask") (remove_unused_layers no)
   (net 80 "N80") (solder_mask_margin 0.102))
  (pad "14" thru_hole circle (at -2.535 2.54 180) (size 1.508 1.508) (drill 1) (layers "*.Cu" "*.Mask") (remove_unused_layers no)
   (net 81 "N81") (solder_mask_margin 0.102))
  (pad "15" thru_hole circle (at -4.815 2.54 180) (size 1.508 1.508) (drill 1) (layers "*.Cu" "*.Mask") (remove_unused_layers no)
   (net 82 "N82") (solder_mask_margin 0.102))
  (pad "S1" thru_hole circle (at -12.495 0 180) (size 4.216 4.216) (drill 3.2) (layers "*.Cu" "*.Mask") (remove_unused_layers no)
   (solder_mask_margin 0.102))
  (pad "S2" thru_hole circle (at 12.495 0 180) (size 4.216 4.216) (drill 3.2) (layers "*.Cu" "*.Mask") (remove_unused_layers no)
   (solder_mask_margin 0.102)))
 (gr_circle (center 235 38) (end 234 38) (stroke (width 0.1) (type default)) (fill none) (layer "Edge.Cuts"))
 (gr_circle (center 45 38) (end 45 39) (stroke (width 0.1) (type default)) (fill none) (layer "Edge.Cuts"))
 (gr_circle (center 45 66) (end 45 65) (stroke (width 0.1) (type default)) (fill none) (layer "Edge.Cuts"))
 (gr_rect (start 40.64 33.02) (end 241.18 71.12) (stroke (width 0.1) (type default)) (fill none) (layer "Edge.Cuts"))
 (gr_circle (center 235 66) (end 236 66) (stroke (width 0.1) (type default)) (fill none) (layer "Edge.Cuts"))
 (segment (start 215.27 60.27) (end 215.27 62.33) (width 0.25) (layer "B.Cu") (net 4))
 (segment (start 192.44675 46.9625) (end 193.52575 45.8835) (width 0.25) (layer "B.Cu") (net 4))
 (segment (start 200.8835 45.8835) (end 215.27 60.27) (width 0.25) (layer "B.Cu") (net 4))
 (segment (start 193.52575 45.8835) (end 200.8835 45.8835) (width 0.25) (layer "B.Cu") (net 4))
 (segment (start 148.215 54.54425) (end 155.75675 47.0025) (width 0.25) (layer "B.Cu") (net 56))
 (segment (start 148.37 63.28) (end 148.215 63.435) (width 0.25) (layer "B.Cu") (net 56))
 (segment (start 148.215 63.435) (end 148.215 54.54425) (width 0.25) (layer "B.Cu") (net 56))
 (segment (start 145.49675 44.4625) (end 145.49675 60.71675) (width 0.25) (layer "B.Cu") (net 57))
 (segment (start 150.755 65.975) (end 150.755 60.895) (width 0.25) (layer "B.Cu") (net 57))
 (segment (start 150.755 65.975) (end 145.675 65.975) (width 0.25) (layer "B.Cu") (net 57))
 (segment (start 145.49675 60.71675) (end 145.675 60.895) (width 0.25) (layer "B.Cu") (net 57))
 (segment (start 145.675 60.895) (end 145.675 65.975) (width 0.25) (layer "B.Cu") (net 57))
 (segment (start 216.595 63.236167) (end 215.986167 63.845) (width 0.25) (layer "B.Cu") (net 5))
 (segment (start 215.986167 63.845) (end 214.015 63.845) (width 0.25) (layer "B.Cu") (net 5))
 (segment (start 190.16675 46.9625) (end 190.16675 44.036563) (width 0.25) (layer "B.Cu") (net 5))
 (segment (start 214.015 63.845) (end 212.5 62.33) (width 0.25) (layer "B.Cu") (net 5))
 (segment (start 200.927333 43.3435) (end 216.595 59.011167) (width 0.25) (layer "B.Cu") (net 5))
 (segment (start 216.595 59.011167) (end 216.595 63.236167) (width 0.25) (layer "B.Cu") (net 5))
 (segment (start 190.859813 43.3435) (end 200.927333 43.3435) (width 0.25) (layer "B.Cu") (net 5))
 (segment (start 190.16675 44.036563) (end 190.859813 43.3435) (width 0.25) (layer "B.Cu") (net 5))
 (segment (start 172.77 62.33) (end 155.9815 45.5415) (width 0.25) (layer "B.Cu") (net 26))
 (segment (start 150.37775 45.5415) (end 148.91675 47.0025) (width 0.25) (layer "B.Cu") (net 26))
 (segment (start 155.9815 45.5415) (end 150.37775 45.5415) (width 0.25) (layer "B.Cu") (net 26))
 (segment (start 158.3835 43.3835) (end 174.095 59.095) (width 0.25) (layer "B.Cu") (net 27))
 (segment (start 146.63675 44.076563) (end 147.329813 43.3835) (width 0.25) (layer "B.Cu") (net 27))
 (segment (start 147.329813 43.3835) (end 158.3835 43.3835) (width 0.25) (layer "B.Cu") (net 27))
 (segment (start 146.63675 47.0025) (end 146.63675 44.076563) (width 0.25) (layer "B.Cu") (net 27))
 (segment (start 171.325 63.655) (end 170 62.33) (width 0.25) (layer "B.Cu") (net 27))
 (segment (start 174.095 59.095) (end 174.095 62.878833) (width 0.25) (layer "B.Cu") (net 27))
 (segment (start 173.318833 63.655) (end 171.325 63.655) (width 0.25) (layer "B.Cu") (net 27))
 (segment (start 174.095 62.878833) (end 173.318833 63.655) (width 0.25) (layer "B.Cu") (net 27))
 (segment (start 113.4815 45.5415) (end 130.27 62.33) (width 0.25) (layer "B.Cu") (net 13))
 (segment (start 107.37775 45.5415) (end 113.4815 45.5415) (width 0.25) (layer "B.Cu") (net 13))
 (segment (start 105.91675 47.0025) (end 107.37775 45.5415) (width 0.25) (layer "B.Cu") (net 13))
 (segment (start 130.938833 63.655) (end 131.715 62.878833) (width 0.25) (layer "B.Cu") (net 12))
 (segment (start 127.5 62.33) (end 128.825 63.655) (width 0.25) (layer "B.Cu") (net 12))
 (segment (start 131.715 62.878833) (end 131.715 61.715) (width 0.25) (layer "B.Cu") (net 12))
 (segment (start 104.4315 43.159813) (end 103.63675 43.954563) (width 0.25) (layer "B.Cu") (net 12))
 (segment (start 128.825 63.655) (end 130.938833 63.655) (width 0.25) (layer "B.Cu") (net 12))
 (segment (start 113.159813 43.159813) (end 104.4315 43.159813) (width 0.25) (layer "B.Cu") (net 12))
 (segment (start 131.715 61.715) (end 113.159813 43.159813) (width 0.25) (layer "B.Cu") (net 12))
 (segment (start 103.63675 43.954563) (end 103.63675 47.0025) (width 0.25) (layer "B.Cu") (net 12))
 (segment (start 61.96 54.79925) (end 61.96 63.5) (width 0.25) (layer "B.Cu") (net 45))
 (segment (start 69.75675 47.0025) (end 61.96 54.79925) (width 0.25) (layer "B.Cu") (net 45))
 (segment (start 62.115 63.345) (end 61.96 63.5) (width 0.25) (layer "B.Cu") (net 45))
 (segment (start 59.42 60.96) (end 59.42 66.04) (width 0.25) (layer "B.Cu") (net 46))
 (segment (start 59.345 60.885) (end 59.42 60.96) (width 0.25) (layer "B.Cu") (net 46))
 (segment (start 59.42 66.04) (end 64.5 66.04) (width 0.25) (layer "B.Cu") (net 46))
 (segment (start 59.49675 60.88325) (end 59.42 60.96) (width 0.25) (layer "B.Cu") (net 46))
 (segment (start 59.49675 44.4625) (end 59.49675 60.88325) (width 0.25) (layer "B.Cu") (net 46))
 (segment (start 64.5 66.04) (end 64.5 60.96) (width 0.25) (layer "B.Cu") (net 46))
 (segment (start 71.3635 45.9235) (end 63.99575 45.9235) (width 0.25) (layer "B.Cu") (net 35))
 (segment (start 87.77 62.33) (end 71.3635 45.9235) (width 0.25) (layer "B.Cu") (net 35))
 (segment (start 63.99575 45.9235) (end 62.91675 47.0025) (width 0.25) (layer "B.Cu") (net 35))
 (segment (start 89.095 63.236167) (end 88.486167 63.845) (width 0.25) (layer "B.Cu") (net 36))
 (segment (start 60.63675 44.076563) (end 61.711813 43.0015) (width 0.25) (layer "B.Cu") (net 36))
 (segment (start 86.515 63.845) (end 85 62.33) (width 0.25) (layer "B.Cu") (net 36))
 (segment (start 70.315333 43.0015) (end 89.095 61.781167) (width 0.25) (layer "B.Cu") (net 36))
 (segment (start 61.711813 43.0015) (end 70.315333 43.0015) (width 0.25) (layer "B.Cu") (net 36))
 (segment (start 88.486167 63.845) (end 86.515 63.845) (width 0.25) (layer "B.Cu") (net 36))
 (segment (start 89.095 61.781167) (end 89.095 63.236167) (width 0.25) (layer "B.Cu") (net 36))
 (segment (start 60.63675 47.0025) (end 60.63675 44.076563) (width 0.25) (layer "B.Cu") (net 36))
 (segment (start 191.5 63.5) (end 191.5 54.74925) (width 0.25) (layer "B.Cu") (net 43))
 (segment (start 191.655 63.345) (end 191.5 63.5) (width 0.25) (layer "B.Cu") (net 43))
 (segment (start 191.5 54.74925) (end 199.28675 46.9625) (width 0.25) (layer "B.Cu") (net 43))
 (segment (start 160 51.7575) (end 115 51.7575) (width 0.25) (layer "F.Cu") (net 1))
 (segment (start 112.95175 51.7575) (end 115 51.7575) (width 0.25) (layer "F.Cu") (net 1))
 (segment (start 202.5 51.7575) (end 231.5 51.7575) (width 0.25) (layer "F.Cu") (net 1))
 (segment (start 194.72675 46.9625) (end 199.52175 51.7575) (width 0.25) (layer "F.Cu") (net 1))
 (segment (start 69.95175 51.7575) (end 65.19675 47.0025) (width 0.25) (layer "F.Cu") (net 1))
 (segment (start 199.52175 51.7575) (end 202.5 51.7575) (width 0.25) (layer "F.Cu") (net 1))
 (segment (start 151.19675 47.0025) (end 155.95175 51.7575) (width 0.25) (layer "F.Cu") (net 1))
 (segment (start 108.19675 47.0025) (end 112.95175 51.7575) (width 0.25) (layer "F.Cu") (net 1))
 (segment (start 115 51.7575) (end 69.95175 51.7575) (width 0.25) (layer "F.Cu") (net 1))
 (segment (start 202.5 51.7575) (end 160 51.7575) (width 0.25) (layer "F.Cu") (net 1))
 (segment (start 155.95175 51.7575) (end 160 51.7575) (width 0.25) (layer "F.Cu") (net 1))
 (segment (start 188.885 60.885) (end 188.96 60.96) (width 0.25) (layer "B.Cu") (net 44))
 (segment (start 194.04 60.96) (end 194.04 66.04) (width 0.25) (layer "B.Cu") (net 44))
 (segment (start 188.96 44.48925) (end 188.96 60.96) (width 0.25) (layer "B.Cu") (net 44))
 (segment (start 188.96 60.96) (end 188.96 66.04) (width 0.25) (layer "B.Cu") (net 44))
 (segment (start 189.02675 44.4225) (end 188.96 44.48925) (width 0.25) (layer "B.Cu") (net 44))
 (segment (start 188.96 66.04) (end 194.04 66.04) (width 0.25) (layer "B.Cu") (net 44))
 (segment (start 67.9975 47.0025) (end 67.47675 47.0025) (width 0.25) (layer "F.Cu") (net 2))
 (segment (start 110.602687 47.0025) (end 117.605187 40) (width 0.25) (layer "F.Cu") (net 2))
 (segment (start 110.47675 47.0025) (end 110.602687 47.0025) (width 0.25) (layer "F.Cu") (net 2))
 (segment (start 162.5 40) (end 120 40) (width 0.25) (layer "F.Cu") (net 2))
 (segment (start 160.605187 40) (end 162.5 40) (width 0.25) (layer "F.Cu") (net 2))
 (segment (start 235.65 51.7575) (end 237.5 51.7575) (width 0.25) (layer "F.Cu") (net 2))
 (segment (start 120 40) (end 75 40) (width 0.25) (layer "F.Cu") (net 2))
 (segment (start 117.605187 40) (end 120 40) (width 0.25) (layer "F.Cu") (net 2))
 (segment (start 204.095187 40) (end 207.5 40) (width 0.25) (layer "F.Cu") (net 2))
 (segment (start 197.00675 46.9625) (end 197.132687 46.9625) (width 0.25) (layer "F.Cu") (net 2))
 (segment (start 75 40) (end 67.9975 47.0025) (width 0.25) (layer "F.Cu") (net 2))
 (segment (start 197.132687 46.9625) (end 204.095187 40) (width 0.25) (layer "F.Cu") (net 2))
 (segment (start 153.47675 47.0025) (end 153.602687 47.0025) (width 0.25) (layer "F.Cu") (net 2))
 (segment (start 223.8925 40) (end 235.65 51.7575) (width 0.25) (layer "F.Cu") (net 2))
 (segment (start 153.602687 47.0025) (end 160.605187 40) (width 0.25) (layer "F.Cu") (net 2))
 (segment (start 162.5 40) (end 223.8925 40) (width 0.25) (layer "F.Cu") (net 2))
 (segment (start 105.295 63.345) (end 105.14 63.5) (width 0.25) (layer "B.Cu") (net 14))
 (segment (start 105.14 54.61925) (end 105.14 63.5) (width 0.25) (layer "B.Cu") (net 14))
 (segment (start 112.75675 47.0025) (end 105.14 54.61925) (width 0.25) (layer "B.Cu") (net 14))
 (segment (start 102.6 60.96) (end 102.6 66.04) (width 0.25) (layer "B.Cu") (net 15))
 (segment (start 107.68 66.04) (end 102.6 66.04) (width 0.25) (layer "B.Cu") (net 15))
 (segment (start 107.68 66.04) (end 107.68 60.96) (width 0.25) (layer "B.Cu") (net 15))
 (segment (start 102.6 60.96) (end 102.49675 60.85675) (width 0.25) (layer "B.Cu") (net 15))
 (segment (start 102.49675 60.85675) (end 102.49675 44.4625) (width 0.25) (layer "B.Cu") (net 15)))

